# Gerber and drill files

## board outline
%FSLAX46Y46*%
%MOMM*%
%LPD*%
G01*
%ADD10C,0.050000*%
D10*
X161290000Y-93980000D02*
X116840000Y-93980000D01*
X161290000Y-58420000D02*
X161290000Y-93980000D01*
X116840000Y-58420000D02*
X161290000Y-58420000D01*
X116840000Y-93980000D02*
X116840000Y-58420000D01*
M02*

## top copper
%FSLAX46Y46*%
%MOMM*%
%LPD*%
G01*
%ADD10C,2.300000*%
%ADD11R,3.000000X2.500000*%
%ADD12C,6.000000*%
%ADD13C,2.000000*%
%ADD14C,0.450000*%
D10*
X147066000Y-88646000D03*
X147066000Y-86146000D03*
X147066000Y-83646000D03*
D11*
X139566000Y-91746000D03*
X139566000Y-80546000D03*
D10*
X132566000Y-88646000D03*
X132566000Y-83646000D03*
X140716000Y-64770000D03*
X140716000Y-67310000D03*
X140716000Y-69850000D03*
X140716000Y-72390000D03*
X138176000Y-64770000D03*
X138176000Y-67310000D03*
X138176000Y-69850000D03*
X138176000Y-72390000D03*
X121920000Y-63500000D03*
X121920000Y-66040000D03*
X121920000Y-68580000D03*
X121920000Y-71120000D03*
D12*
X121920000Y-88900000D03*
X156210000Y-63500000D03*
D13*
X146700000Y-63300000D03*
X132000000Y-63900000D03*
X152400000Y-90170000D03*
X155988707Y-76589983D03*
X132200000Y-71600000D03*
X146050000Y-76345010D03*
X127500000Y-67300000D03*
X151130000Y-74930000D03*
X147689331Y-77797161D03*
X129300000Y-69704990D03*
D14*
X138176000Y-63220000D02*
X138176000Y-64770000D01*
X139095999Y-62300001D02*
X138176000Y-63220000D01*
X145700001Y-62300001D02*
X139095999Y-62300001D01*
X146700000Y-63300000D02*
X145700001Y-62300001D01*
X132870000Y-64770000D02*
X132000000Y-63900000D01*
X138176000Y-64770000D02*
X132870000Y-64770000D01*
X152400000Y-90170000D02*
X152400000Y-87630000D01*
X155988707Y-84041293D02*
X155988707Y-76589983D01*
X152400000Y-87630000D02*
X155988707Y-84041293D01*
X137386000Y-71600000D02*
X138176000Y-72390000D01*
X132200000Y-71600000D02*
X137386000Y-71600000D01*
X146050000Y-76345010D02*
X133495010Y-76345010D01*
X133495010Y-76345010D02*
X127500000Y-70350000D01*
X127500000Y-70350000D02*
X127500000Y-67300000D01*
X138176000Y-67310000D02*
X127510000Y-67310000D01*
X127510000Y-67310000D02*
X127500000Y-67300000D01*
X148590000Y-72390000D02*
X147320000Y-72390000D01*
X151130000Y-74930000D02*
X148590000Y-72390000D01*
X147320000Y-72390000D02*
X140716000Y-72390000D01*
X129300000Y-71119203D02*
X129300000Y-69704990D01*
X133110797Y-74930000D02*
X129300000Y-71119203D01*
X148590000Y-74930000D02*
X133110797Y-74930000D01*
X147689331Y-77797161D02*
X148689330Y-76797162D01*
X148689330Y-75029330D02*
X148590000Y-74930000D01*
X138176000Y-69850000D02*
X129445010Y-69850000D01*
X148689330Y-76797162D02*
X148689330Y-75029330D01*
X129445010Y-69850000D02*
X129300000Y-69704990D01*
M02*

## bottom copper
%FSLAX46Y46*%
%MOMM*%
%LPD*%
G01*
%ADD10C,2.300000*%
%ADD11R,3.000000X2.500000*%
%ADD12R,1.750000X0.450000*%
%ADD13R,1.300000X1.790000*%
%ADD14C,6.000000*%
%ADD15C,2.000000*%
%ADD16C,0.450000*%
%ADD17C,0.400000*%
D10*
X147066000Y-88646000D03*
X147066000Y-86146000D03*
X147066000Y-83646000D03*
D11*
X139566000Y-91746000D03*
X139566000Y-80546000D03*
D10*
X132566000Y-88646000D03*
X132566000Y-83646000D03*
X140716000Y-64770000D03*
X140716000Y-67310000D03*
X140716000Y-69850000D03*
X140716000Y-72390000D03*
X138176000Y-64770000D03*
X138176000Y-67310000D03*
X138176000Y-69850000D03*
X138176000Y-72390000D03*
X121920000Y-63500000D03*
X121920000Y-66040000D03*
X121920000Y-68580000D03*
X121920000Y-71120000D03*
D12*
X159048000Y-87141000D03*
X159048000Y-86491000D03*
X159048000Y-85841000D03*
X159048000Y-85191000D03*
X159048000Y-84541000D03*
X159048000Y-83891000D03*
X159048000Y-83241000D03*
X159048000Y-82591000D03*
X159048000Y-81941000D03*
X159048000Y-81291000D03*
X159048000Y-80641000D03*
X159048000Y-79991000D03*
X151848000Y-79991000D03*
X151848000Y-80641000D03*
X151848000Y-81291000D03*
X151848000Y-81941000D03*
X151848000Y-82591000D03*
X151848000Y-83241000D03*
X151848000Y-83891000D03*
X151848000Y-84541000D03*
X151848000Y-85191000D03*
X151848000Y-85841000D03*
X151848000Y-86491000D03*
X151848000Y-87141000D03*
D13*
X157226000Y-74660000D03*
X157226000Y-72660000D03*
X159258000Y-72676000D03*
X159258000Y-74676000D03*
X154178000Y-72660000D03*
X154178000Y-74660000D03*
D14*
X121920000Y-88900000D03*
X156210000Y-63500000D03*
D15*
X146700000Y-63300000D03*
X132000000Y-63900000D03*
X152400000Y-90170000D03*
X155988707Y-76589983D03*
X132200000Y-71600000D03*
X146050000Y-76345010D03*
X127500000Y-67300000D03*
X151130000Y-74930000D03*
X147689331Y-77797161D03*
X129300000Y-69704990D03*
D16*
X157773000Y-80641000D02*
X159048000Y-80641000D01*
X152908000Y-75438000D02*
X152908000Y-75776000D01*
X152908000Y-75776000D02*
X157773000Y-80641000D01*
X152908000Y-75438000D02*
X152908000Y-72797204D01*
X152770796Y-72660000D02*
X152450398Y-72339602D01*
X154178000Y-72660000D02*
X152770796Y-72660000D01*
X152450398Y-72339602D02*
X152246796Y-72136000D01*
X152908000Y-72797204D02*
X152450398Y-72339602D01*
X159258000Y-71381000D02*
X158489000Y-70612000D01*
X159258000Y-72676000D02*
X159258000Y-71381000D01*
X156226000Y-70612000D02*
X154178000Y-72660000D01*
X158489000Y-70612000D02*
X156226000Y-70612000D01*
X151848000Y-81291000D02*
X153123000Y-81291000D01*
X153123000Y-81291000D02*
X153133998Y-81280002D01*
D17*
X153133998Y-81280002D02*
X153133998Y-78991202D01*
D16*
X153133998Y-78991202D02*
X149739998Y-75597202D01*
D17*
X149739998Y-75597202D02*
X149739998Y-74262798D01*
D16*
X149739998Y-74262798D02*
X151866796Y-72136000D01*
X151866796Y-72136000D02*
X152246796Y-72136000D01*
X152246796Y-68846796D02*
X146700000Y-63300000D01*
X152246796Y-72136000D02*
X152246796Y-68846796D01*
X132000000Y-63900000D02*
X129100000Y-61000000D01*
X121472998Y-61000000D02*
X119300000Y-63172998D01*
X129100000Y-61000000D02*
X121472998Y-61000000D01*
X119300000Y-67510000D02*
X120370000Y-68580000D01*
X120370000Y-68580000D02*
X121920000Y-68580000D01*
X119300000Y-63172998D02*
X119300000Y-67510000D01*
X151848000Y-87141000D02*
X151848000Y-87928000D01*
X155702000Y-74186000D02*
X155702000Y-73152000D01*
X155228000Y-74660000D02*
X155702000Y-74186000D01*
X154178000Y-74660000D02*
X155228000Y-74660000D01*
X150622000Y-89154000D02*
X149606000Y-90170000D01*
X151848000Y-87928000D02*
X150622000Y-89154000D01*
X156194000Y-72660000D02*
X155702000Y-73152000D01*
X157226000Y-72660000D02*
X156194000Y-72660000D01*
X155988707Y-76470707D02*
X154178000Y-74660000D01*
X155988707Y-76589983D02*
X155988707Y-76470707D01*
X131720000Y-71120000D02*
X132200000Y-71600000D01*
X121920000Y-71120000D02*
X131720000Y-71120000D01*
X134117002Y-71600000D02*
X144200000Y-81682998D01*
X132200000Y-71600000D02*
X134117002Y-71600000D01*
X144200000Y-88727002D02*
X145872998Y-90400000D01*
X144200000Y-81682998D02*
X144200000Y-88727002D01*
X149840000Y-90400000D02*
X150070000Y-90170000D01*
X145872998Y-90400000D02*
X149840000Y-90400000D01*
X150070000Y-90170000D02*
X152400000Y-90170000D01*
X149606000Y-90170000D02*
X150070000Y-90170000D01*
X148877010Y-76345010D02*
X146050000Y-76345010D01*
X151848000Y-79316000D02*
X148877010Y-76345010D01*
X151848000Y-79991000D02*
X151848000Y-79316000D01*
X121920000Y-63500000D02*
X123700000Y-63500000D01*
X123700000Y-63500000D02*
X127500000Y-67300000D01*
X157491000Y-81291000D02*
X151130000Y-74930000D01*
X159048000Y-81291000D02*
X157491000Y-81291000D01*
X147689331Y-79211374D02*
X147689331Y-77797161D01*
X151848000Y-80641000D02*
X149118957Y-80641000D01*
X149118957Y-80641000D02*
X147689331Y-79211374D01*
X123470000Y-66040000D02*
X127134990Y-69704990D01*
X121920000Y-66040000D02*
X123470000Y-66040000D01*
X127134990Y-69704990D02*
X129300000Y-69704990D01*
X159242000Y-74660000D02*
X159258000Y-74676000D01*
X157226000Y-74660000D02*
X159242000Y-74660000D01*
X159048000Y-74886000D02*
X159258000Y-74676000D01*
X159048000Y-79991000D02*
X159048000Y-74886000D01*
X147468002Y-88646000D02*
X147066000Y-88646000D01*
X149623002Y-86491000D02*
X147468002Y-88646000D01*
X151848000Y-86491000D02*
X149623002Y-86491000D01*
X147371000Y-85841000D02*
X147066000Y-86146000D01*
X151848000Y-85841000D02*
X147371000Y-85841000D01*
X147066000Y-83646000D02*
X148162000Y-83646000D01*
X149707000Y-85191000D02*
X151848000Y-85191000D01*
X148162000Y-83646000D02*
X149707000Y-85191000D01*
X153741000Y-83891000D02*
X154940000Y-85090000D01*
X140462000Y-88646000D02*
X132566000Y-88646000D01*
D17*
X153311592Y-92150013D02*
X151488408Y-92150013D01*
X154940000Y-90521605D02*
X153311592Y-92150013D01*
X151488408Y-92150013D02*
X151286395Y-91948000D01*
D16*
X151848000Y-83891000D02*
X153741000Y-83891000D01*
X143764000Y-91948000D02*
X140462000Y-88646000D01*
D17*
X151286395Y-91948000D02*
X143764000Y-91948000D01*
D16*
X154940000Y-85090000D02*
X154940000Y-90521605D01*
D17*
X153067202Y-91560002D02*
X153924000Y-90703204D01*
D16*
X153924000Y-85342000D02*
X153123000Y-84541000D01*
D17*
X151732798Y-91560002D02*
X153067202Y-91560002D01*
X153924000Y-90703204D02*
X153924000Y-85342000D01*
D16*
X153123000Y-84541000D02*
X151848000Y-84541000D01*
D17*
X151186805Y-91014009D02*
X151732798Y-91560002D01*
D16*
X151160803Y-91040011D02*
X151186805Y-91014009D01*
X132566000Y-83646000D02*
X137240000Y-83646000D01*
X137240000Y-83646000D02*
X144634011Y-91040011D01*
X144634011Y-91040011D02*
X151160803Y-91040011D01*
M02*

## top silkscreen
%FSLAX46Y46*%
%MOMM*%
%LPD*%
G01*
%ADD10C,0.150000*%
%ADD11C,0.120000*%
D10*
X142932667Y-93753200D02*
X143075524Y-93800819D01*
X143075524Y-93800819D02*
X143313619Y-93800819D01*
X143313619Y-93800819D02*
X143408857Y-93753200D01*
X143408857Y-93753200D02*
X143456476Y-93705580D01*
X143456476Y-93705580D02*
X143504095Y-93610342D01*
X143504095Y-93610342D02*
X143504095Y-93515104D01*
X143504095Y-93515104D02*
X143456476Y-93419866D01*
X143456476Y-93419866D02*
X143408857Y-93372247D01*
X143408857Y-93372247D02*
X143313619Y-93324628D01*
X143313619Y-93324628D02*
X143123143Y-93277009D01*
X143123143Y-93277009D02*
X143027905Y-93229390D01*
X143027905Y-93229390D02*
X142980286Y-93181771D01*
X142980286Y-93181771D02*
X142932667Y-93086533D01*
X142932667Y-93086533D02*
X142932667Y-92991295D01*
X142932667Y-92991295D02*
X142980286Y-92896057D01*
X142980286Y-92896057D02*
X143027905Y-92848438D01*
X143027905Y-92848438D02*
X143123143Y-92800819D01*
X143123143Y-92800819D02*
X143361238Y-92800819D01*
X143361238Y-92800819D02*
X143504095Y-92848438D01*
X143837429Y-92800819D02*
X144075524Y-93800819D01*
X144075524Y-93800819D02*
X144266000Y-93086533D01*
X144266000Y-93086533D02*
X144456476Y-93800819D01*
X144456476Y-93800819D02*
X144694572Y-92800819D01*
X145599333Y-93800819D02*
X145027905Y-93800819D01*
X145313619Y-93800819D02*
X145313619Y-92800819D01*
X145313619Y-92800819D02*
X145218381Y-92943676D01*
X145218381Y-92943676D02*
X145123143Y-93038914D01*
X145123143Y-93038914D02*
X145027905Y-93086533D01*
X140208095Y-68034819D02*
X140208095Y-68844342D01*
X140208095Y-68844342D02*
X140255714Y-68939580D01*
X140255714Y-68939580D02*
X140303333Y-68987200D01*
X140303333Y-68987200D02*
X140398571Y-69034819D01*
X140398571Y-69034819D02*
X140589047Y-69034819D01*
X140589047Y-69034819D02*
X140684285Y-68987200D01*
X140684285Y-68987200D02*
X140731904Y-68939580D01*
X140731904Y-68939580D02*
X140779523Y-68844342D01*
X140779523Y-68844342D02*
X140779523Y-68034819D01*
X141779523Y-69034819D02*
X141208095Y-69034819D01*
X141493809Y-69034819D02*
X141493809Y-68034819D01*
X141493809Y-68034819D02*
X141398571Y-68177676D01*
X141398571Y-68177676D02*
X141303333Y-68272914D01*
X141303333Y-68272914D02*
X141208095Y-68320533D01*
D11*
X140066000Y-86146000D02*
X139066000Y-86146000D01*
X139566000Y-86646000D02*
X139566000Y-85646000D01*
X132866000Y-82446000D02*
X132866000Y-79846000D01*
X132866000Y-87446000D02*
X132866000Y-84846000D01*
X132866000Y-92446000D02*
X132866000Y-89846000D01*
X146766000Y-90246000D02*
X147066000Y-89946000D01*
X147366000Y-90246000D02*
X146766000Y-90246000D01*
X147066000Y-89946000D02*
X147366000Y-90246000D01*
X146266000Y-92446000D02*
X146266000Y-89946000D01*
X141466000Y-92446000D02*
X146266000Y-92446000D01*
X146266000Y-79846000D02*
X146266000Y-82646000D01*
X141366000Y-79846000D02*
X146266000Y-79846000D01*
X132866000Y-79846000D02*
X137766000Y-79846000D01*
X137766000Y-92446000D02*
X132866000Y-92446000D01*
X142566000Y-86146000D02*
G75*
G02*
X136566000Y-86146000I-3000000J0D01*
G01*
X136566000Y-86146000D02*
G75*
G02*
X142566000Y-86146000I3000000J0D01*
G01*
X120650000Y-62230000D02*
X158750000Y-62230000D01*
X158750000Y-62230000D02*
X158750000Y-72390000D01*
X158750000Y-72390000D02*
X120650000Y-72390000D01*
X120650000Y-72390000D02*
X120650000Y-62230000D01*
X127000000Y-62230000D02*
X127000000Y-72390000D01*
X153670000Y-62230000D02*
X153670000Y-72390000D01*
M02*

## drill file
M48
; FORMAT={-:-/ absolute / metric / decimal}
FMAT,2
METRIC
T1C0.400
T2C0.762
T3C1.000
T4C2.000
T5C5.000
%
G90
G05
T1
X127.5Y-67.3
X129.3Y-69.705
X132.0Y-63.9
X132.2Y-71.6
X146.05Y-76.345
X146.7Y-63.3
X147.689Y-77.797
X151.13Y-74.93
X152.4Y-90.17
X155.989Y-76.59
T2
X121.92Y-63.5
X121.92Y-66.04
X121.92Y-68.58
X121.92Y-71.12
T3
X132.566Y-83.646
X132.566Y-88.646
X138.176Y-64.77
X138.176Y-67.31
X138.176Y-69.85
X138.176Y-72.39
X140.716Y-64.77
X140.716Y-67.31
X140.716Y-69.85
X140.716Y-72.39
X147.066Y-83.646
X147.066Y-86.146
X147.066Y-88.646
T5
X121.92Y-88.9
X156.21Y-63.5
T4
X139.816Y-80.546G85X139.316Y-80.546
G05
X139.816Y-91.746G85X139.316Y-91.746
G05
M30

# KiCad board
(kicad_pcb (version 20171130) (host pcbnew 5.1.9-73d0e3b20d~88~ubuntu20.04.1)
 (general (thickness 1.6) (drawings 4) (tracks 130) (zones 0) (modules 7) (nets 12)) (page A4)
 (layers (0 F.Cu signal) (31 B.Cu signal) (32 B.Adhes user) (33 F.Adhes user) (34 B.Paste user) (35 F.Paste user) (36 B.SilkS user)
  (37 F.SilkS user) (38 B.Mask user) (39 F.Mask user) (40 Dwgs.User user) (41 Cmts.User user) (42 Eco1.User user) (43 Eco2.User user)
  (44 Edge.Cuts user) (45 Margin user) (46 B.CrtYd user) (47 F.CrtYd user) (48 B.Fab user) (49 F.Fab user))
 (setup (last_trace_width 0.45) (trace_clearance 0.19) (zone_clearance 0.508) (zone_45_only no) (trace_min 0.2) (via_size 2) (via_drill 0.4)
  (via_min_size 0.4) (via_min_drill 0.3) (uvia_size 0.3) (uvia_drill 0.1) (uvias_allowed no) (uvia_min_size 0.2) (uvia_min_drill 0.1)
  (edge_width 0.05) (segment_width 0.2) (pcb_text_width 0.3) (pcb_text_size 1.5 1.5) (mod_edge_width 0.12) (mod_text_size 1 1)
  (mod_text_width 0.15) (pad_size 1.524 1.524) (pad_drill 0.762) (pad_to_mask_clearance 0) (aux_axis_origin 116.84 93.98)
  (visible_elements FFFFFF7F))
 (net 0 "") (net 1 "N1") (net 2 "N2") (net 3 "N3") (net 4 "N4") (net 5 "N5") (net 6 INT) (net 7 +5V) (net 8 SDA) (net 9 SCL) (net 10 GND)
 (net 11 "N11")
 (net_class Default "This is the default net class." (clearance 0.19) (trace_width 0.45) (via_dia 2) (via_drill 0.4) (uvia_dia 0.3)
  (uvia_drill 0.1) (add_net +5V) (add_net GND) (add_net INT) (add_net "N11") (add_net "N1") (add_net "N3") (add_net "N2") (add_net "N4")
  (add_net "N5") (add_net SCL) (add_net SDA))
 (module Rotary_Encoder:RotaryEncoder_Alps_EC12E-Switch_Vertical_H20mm (layer F.Cu) (at 147.066 88.646 180)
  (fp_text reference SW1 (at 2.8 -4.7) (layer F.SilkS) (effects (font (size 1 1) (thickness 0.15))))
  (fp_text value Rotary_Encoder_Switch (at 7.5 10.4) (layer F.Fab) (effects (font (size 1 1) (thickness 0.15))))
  (fp_line (start 7 2.5) (end 8 2.5) (layer F.SilkS) (width 0.12))
  (fp_line (start 7.5 2) (end 7.5 3) (layer F.SilkS) (width 0.12))
  (fp_line (start 14.2 6.2) (end 14.2 8.8) (layer F.SilkS) (width 0.12))
  (fp_line (start 14.2 1.2) (end 14.2 3.8) (layer F.SilkS) (width 0.12))
  (fp_line (start 14.2 -3.8) (end 14.2 -1.2) (layer F.SilkS) (width 0.12))
  (fp_line (start 0.3 -1.6) (end 0 -1.3) (layer F.SilkS) (width 0.12))
  (fp_line (start -0.3 -1.6) (end 0.3 -1.6) (layer F.SilkS) (width 0.12))
  (fp_line (start 0 -1.3) (end -0.3 -1.6) (layer F.SilkS) (width 0.12))
  (fp_line (start 0.8 -3.8) (end 0.8 -1.3) (layer F.SilkS) (width 0.12))
  (fp_line (start 5.6 -3.8) (end 0.8 -3.8) (layer F.SilkS) (width 0.12))
  (fp_line (start 0.8 8.8) (end 0.8 6) (layer F.SilkS) (width 0.12))
  (fp_line (start 5.7 8.8) (end 0.8 8.8) (layer F.SilkS) (width 0.12))
  (fp_line (start 14.2 8.8) (end 9.3 8.8) (layer F.SilkS) (width 0.12))
  (fp_line (start 9.3 -3.8) (end 14.2 -3.8) (layer F.SilkS) (width 0.12))
  (fp_circle (center 7.5 2.5) (end 10.5 2.5) (layer F.SilkS) (width 0.12))
  (pad A thru_hole circle (at 0 0 180) (size 2.3 2.3) (drill 1) (layers *.Cu *.Mask) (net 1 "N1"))
  (pad C thru_hole circle (at 0 2.5 180) (size 2.3 2.3) (drill 1) (layers *.Cu *.Mask) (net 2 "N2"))
  (pad B thru_hole circle (at 0 5 180) (size 2.3 2.3) (drill 1) (layers *.Cu *.Mask) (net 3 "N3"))
  (pad MP thru_hole rect (at 7.5 -3.1 180) (size 3 2.5) (drill oval 2.5 2) (layers *.Cu *.Mask))
  (pad MP thru_hole rect (at 7.5 8.1 180) (size 3 2.5) (drill oval 2.5 2) (layers *.Cu *.Mask))
  (pad S1 thru_hole circle (at 14.5 0 180) (size 2.3 2.3) (drill 1) (layers *.Cu *.Mask) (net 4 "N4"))
  (pad S2 thru_hole circle (at 14.5 5 180) (size 2.3 2.3) (drill 1) (layers *.Cu *.Mask) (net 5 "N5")))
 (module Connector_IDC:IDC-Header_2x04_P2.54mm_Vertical (layer B.Cu) (at 138.176 72.39)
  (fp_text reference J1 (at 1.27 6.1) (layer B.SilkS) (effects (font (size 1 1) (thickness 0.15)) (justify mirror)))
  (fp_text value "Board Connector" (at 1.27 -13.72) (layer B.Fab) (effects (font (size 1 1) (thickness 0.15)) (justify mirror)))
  (pad 8 thru_hole circle (at 2.54 -7.62) (size 2.3 2.3) (drill 1) (layers *.Cu *.Mask))
  (pad 6 thru_hole circle (at 2.54 -5.08) (size 2.3 2.3) (drill 1) (layers *.Cu *.Mask))
  (pad 4 thru_hole circle (at 2.54 -2.54) (size 2.3 2.3) (drill 1) (layers *.Cu *.Mask))
  (pad 2 thru_hole circle (at 2.54 0) (size 2.3 2.3) (drill 1) (layers *.Cu *.Mask) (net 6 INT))
  (pad 7 thru_hole circle (at 0 -7.62) (size 2.3 2.3) (drill 1) (layers *.Cu *.Mask) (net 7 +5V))
  (pad 5 thru_hole circle (at 0 -5.08) (size 2.3 2.3) (drill 1) (layers *.Cu *.Mask) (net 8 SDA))
  (pad 3 thru_hole circle (at 0 -2.54) (size 2.3 2.3) (drill 1) (layers *.Cu *.Mask) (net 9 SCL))
  (pad 1 thru_hole circle (at 0 0) (size 2.3 2.3) (drill 1) (layers *.Cu *.Mask) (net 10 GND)))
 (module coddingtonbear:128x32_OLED (layer F.Cu) (at 129.54 68.58)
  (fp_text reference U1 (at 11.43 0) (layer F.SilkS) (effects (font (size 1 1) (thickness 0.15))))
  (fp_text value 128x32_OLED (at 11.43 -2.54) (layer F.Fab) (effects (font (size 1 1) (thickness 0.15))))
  (fp_line (start -8.89 -6.35) (end 29.21 -6.35) (layer F.SilkS) (width 0.12))
  (fp_line (start 29.21 -6.35) (end 29.21 3.81) (layer F.SilkS) (width 0.12))
  (fp_line (start 29.21 3.81) (end -8.89 3.81) (layer F.SilkS) (width 0.12))
  (fp_line (start -8.89 3.81) (end -8.89 -6.35) (layer F.SilkS) (width 0.12))
  (fp_line (start -2.54 -6.35) (end -2.54 3.81) (layer F.SilkS) (width 0.12))
  (fp_line (start 24.13 -6.35) (end 24.13 3.81) (layer F.SilkS) (width 0.12))
  (pad 4 thru_hole circle (at -7.62 -5.08) (size 2.3 2.3) (drill 0.762) (layers *.Cu *.Mask) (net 8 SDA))
  (pad 3 thru_hole circle (at -7.62 -2.54) (size 2.3 2.3) (drill 0.762) (layers *.Cu *.Mask) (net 9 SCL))
  (pad 2 thru_hole circle (at -7.62 0) (size 2.3 2.3) (drill 0.762) (layers *.Cu *.Mask) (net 7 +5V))
  (pad 1 thru_hole circle (at -7.62 2.54) (size 2.3 2.3) (drill 0.762) (layers *.Cu *.Mask) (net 10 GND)))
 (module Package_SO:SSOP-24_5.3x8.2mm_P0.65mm (layer B.Cu) (at 155.448 83.566)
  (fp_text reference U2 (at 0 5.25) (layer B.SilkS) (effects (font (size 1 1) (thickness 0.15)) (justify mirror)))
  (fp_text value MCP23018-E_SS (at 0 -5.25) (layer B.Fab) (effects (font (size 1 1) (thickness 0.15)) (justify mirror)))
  (pad 24 smd rect (at 3.6 3.575) (size 1.75 0.45) (layers B.Cu B.Paste B.Mask))
  (pad 23 smd rect (at 3.6 2.925) (size 1.75 0.45) (layers B.Cu B.Paste B.Mask))
  (pad 22 smd rect (at 3.6 2.275) (size 1.75 0.45) (layers B.Cu B.Paste B.Mask))
  (pad 21 smd rect (at 3.6 1.625) (size 1.75 0.45) (layers B.Cu B.Paste B.Mask))
  (pad 20 smd rect (at 3.6 0.975) (size 1.75 0.45) (layers B.Cu B.Paste B.Mask))
  (pad 19 smd rect (at 3.6 0.325) (size 1.75 0.45) (layers B.Cu B.Paste B.Mask))
  (pad 18 smd rect (at 3.6 -0.325) (size 1.75 0.45) (layers B.Cu B.Paste B.Mask))
  (pad 17 smd rect (at 3.6 -0.975) (size 1.75 0.45) (layers B.Cu B.Paste B.Mask))
  (pad 16 smd rect (at 3.6 -1.625) (size 1.75 0.45) (layers B.Cu B.Paste B.Mask))
  (pad 15 smd rect (at 3.6 -2.275) (size 1.75 0.45) (layers B.Cu B.Paste B.Mask) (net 6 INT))
  (pad 14 smd rect (at 3.6 -2.925) (size 1.75 0.45) (layers B.Cu B.Paste B.Mask) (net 7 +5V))
  (pad 13 smd rect (at 3.6 -3.575) (size 1.75 0.45) (layers B.Cu B.Paste B.Mask) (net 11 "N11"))
  (pad 12 smd rect (at -3.6 -3.575) (size 1.75 0.45) (layers B.Cu B.Paste B.Mask) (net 8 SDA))
  (pad 11 smd rect (at -3.6 -2.925) (size 1.75 0.45) (layers B.Cu B.Paste B.Mask) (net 9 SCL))
  (pad 10 smd rect (at -3.6 -2.275) (size 1.75 0.45) (layers B.Cu B.Paste B.Mask) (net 7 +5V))
  (pad 9 smd rect (at -3.6 -1.625) (size 1.75 0.45) (layers B.Cu B.Paste B.Mask))
  (pad 8 smd rect (at -3.6 -0.975) (size 1.75 0.45) (layers B.Cu B.Paste B.Mask))
  (pad 7 smd rect (at -3.6 -0.325) (size 1.75 0.45) (layers B.Cu B.Paste B.Mask))
  (pad 6 smd rect (at -3.6 0.325) (size 1.75 0.45) (layers B.Cu B.Paste B.Mask) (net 4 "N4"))
  (pad 5 smd rect (at -3.6 0.975) (size 1.75 0.45) (layers B.Cu B.Paste B.Mask) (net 5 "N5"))
  (pad 4 smd rect (at -3.6 1.625) (size 1.75 0.45) (layers B.Cu B.Paste B.Mask) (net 3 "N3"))
  (pad 3 smd rect (at -3.6 2.275) (size 1.75 0.45) (layers B.Cu B.Paste B.Mask) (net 2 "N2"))
  (pad 2 smd rect (at -3.6 2.925) (size 1.75 0.45) (layers B.Cu B.Paste B.Mask) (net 1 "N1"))
  (pad 1 smd rect (at -3.6 3.575) (size 1.75 0.45) (layers B.Cu B.Paste B.Mask) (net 10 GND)))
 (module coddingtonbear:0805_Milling (layer B.Cu) (at 157.226 73.66 90)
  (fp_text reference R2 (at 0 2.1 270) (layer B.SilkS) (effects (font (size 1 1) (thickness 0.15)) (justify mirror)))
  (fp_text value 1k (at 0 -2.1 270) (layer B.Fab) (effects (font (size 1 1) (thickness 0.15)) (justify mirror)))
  (pad 1 smd rect (at -1 0 90) (size 1.79 1.3) (layers B.Cu B.Paste B.Mask) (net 11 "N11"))
  (pad 2 smd rect (at 1 0 90) (size 1.79 1.3) (layers B.Cu B.Paste B.Mask) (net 10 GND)))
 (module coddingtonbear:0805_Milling (layer B.Cu) (at 159.258 73.676 270)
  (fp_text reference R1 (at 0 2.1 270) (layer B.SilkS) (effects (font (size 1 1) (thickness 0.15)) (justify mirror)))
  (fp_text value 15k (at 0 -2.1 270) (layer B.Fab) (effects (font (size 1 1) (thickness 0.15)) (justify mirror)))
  (pad 1 smd rect (at -1 0 270) (size 1.79 1.3) (layers B.Cu B.Paste B.Mask) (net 7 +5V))
  (pad 2 smd rect (at 1 0 270) (size 1.79 1.3) (layers B.Cu B.Paste B.Mask) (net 11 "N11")))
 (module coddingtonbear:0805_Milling (layer B.Cu) (at 154.178 73.66 270)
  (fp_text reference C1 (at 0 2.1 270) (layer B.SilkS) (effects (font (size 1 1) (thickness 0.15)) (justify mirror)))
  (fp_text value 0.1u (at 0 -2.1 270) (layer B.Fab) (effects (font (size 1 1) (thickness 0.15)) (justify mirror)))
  (pad 1 smd rect (at -1 0 270) (size 1.79 1.3) (layers B.Cu B.Paste B.Mask) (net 7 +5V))
  (pad 2 smd rect (at 1 0 270) (size 1.79 1.3) (layers B.Cu B.Paste B.Mask) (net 10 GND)))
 (gr_line (start 161.29 93.98) (end 116.84 93.98) (layer Edge.Cuts) (width 0.05))
 (gr_line (start 161.29 58.42) (end 161.29 93.98) (layer Edge.Cuts) (width 0.05))
 (gr_line (start 116.84 58.42) (end 161.29 58.42) (layer Edge.Cuts) (width 0.05))
 (gr_line (start 116.84 93.98) (end 116.84 58.42) (layer Edge.Cuts) (width 0.05))
 (via (at 121.92 88.9) (size 6) (drill 5) (layers F.Cu B.Cu) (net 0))
 (via (at 156.21 63.5) (size 6) (drill 5) (layers F.Cu B.Cu) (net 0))
 (segment (start 157.773 80.641) (end 159.048 80.641) (width 0.45) (layer B.Cu) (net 7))
 (segment (start 152.908 75.438) (end 152.908 75.776) (width 0.45) (layer B.Cu) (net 7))
 (segment (start 152.908 75.776) (end 157.773 80.641) (width 0.45) (layer B.Cu) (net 7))
 (segment (start 152.908 75.438) (end 152.908 72.797204) (width 0.45) (layer B.Cu) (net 7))
 (segment (start 152.770796 72.66) (end 152.450398 72.339602) (width 0.45) (layer B.Cu) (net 7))
 (segment (start 154.178 72.66) (end 152.770796 72.66) (width 0.45) (layer B.Cu) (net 7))
 (segment (start 152.450398 72.339602) (end 152.246796 72.136) (width 0.45) (layer B.Cu) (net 7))
 (segment (start 152.908 72.797204) (end 152.450398 72.339602) (width 0.45) (layer B.Cu) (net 7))
 (segment (start 159.258 71.381) (end 158.489 70.612) (width 0.45) (layer B.Cu) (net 7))
 (segment (start 159.258 72.676) (end 159.258 71.381) (width 0.45) (layer B.Cu) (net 7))
 (segment (start 156.226 70.612) (end 154.178 72.66) (width 0.45) (layer B.Cu) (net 7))
 (segment (start 158.489 70.612) (end 156.226 70.612) (width 0.45) (layer B.Cu) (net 7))
 (segment (start 151.848 81.291) (end 153.123 81.291) (width 0.45) (layer B.Cu) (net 7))
 (segment (start 153.123 81.291) (end 153.133998 81.280002) (width 0.45) (layer B.Cu) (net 7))
 (segment (start 153.133998 81.280002) (end 153.133998 78.991202) (width 0.4) (layer B.Cu) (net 7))
 (segment (start 153.133998 78.991202) (end 149.739998 75.597202) (width 0.45) (layer B.Cu) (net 7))
 (segment (start 149.739998 75.597202) (end 149.739998 74.262798) (width 0.4) (layer B.Cu) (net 7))
 (segment (start 149.739998 74.262798) (end 151.866796 72.136) (width 0.45) (layer B.Cu) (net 7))
 (segment (start 151.866796 72.136) (end 152.246796 72.136) (width 0.45) (layer B.Cu) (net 7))
 (via (at 146.7 63.3) (size 2) (drill 0.4) (layers F.Cu B.Cu) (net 7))
 (segment (start 152.246796 68.846796) (end 146.7 63.3) (width 0.45) (layer B.Cu) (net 7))
 (segment (start 152.246796 72.136) (end 152.246796 68.846796) (width 0.45) (layer B.Cu) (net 7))
 (segment (start 138.176 63.22) (end 138.176 64.77) (width 0.45) (layer F.Cu) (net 7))
 (segment (start 139.095999 62.300001) (end 138.176 63.22) (width 0.45) (layer F.Cu) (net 7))
 (segment (start 145.700001 62.300001) (end 139.095999 62.300001) (width 0.45) (layer F.Cu) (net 7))
 (segment (start 146.7 63.3) (end 145.700001 62.300001) (width 0.45) (layer F.Cu) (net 7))
 (segment (start 132.87 64.77) (end 132 63.9) (width 0.45) (layer F.Cu) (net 7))
 (via (at 132 63.9) (size 2) (drill 0.4) (layers F.Cu B.Cu) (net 7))
 (segment (start 138.176 64.77) (end 132.87 64.77) (width 0.45) (layer F.Cu) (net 7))
 (segment (start 132 63.9) (end 129.1 61) (width 0.45) (layer B.Cu) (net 7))
 (segment (start 121.472998 61) (end 119.3 63.172998) (width 0.45) (layer B.Cu) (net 7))
 (segment (start 129.1 61) (end 121.472998 61) (width 0.45) (layer B.Cu) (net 7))
 (segment (start 119.3 67.51) (end 120.37 68.58) (width 0.45) (layer B.Cu) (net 7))
 (segment (start 120.37 68.58) (end 121.92 68.58) (width 0.45) (layer B.Cu) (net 7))
 (segment (start 119.3 63.172998) (end 119.3 67.51) (width 0.45) (layer B.Cu) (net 7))
 (segment (start 151.848 87.141) (end 151.848 87.928) (width 0.45) (layer B.Cu) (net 10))
 (segment (start 155.702 74.186) (end 155.702 73.152) (width 0.45) (layer B.Cu) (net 10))
 (segment (start 155.228 74.66) (end 155.702 74.186) (width 0.45) (layer B.Cu) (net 10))
 (segment (start 154.178 74.66) (end 155.228 74.66) (width 0.45) (layer B.Cu) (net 10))
 (segment (start 150.622 89.154) (end 149.606 90.17) (width 0.45) (layer B.Cu) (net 10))
 (segment (start 151.848 87.928) (end 150.622 89.154) (width 0.45) (layer B.Cu) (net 10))
 (segment (start 156.194 72.66) (end 155.702 73.152) (width 0.45) (layer B.Cu) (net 10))
 (segment (start 157.226 72.66) (end 156.194 72.66) (width 0.45) (layer B.Cu) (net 10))
 (via (at 152.4 90.17) (size 2) (drill 0.4) (layers F.Cu B.Cu) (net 10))
 (segment (start 152.4 90.17) (end 152.4 87.63) (width 0.45) (layer F.Cu) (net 10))
 (via (at 155.988707 76.589983) (size 2) (drill 0.4) (layers F.Cu B.Cu) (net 10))
 (segment (start 155.988707 84.041293) (end 155.988707 76.589983) (width 0.45) (layer F.Cu) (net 10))
 (segment (start 152.4 87.63) (end 155.988707 84.041293) (width 0.45) (layer F.Cu) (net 10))
 (segment (start 155.988707 76.470707) (end 154.178 74.66) (width 0.45) (layer B.Cu) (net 10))
 (segment (start 155.988707 76.589983) (end 155.988707 76.470707) (width 0.45) (layer B.Cu) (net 10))
 (segment (start 131.72 71.12) (end 132.2 71.6) (width 0.45) (layer B.Cu) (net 10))
 (segment (start 121.92 71.12) (end 131.72 71.12) (width 0.45) (layer B.Cu) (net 10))
 (via (at 132.2 71.6) (size 2) (drill 0.4) (layers F.Cu B.Cu) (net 10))
 (segment (start 137.386 71.6) (end 138.176 72.39) (width 0.45) (layer F.Cu) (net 10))
 (segment (start 132.2 71.6) (end 137.386 71.6) (width 0.45) (layer F.Cu) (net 10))
 (segment (start 134.117002 71.6) (end 144.2 81.682998) (width 0.45) (layer B.Cu) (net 10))
 (segment (start 132.2 71.6) (end 134.117002 71.6) (width 0.45) (layer B.Cu) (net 10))
 (segment (start 144.2 88.727002) (end 145.872998 90.4) (width 0.45) (layer B.Cu) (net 10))
 (segment (start 144.2 81.682998) (end 144.2 88.727002) (width 0.45) (layer B.Cu) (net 10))
 (segment (start 149.84 90.4) (end 150.07 90.17) (width 0.45) (layer B.Cu) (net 10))
 (segment (start 145.872998 90.4) (end 149.84 90.4) (width 0.45) (layer B.Cu) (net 10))
 (segment (start 150.07 90.17) (end 152.4 90.17) (width 0.45) (layer B.Cu) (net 10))
 (segment (start 149.606 90.17) (end 150.07 90.17) (width 0.45) (layer B.Cu) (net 10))
 (segment (start 148.87701 76.34501) (end 146.05 76.34501) (width 0.45) (layer B.Cu) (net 8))
 (segment (start 151.848 79.316) (end 148.87701 76.34501) (width 0.45) (layer B.Cu) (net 8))
 (segment (start 151.848 79.991) (end 151.848 79.316) (width 0.45) (layer B.Cu) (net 8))
 (via (at 146.05 76.34501) (size 2) (drill 0.4) (layers F.Cu B.Cu) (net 8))
 (segment (start 121.92 63.5) (end 123.7 63.5) (width 0.45) (layer B.Cu) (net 8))
 (segment (start 123.7 63.5) (end 127.5 67.3) (width 0.45) (layer B.Cu) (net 8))
 (segment (start 146.05 76.34501) (end 133.49501 76.34501) (width 0.45) (layer F.Cu) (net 8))
 (via (at 127.5 67.3) (size 2) (drill 0.4) (layers F.Cu B.Cu) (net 8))
 (segment (start 133.49501 76.34501) (end 127.5 70.35) (width 0.45) (layer F.Cu) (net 8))
 (segment (start 127.5 70.35) (end 127.5 67.3) (width 0.45) (layer F.Cu) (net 8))
 (segment (start 138.176 67.31) (end 127.51 67.31) (width 0.45) (layer F.Cu) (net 8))
 (segment (start 127.51 67.31) (end 127.5 67.3) (width 0.45) (layer F.Cu) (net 8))
 (via (at 151.13 74.93) (size 2) (drill 0.4) (layers F.Cu B.Cu) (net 6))
 (segment (start 157.491 81.291) (end 151.13 74.93) (width 0.45) (layer B.Cu) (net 6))
 (segment (start 159.048 81.291) (end 157.491 81.291) (width 0.45) (layer B.Cu) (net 6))
 (segment (start 148.59 72.39) (end 147.32 72.39) (width 0.45) (layer F.Cu) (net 6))
 (segment (start 151.13 74.93) (end 148.59 72.39) (width 0.45) (layer F.Cu) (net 6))
 (segment (start 147.32 72.39) (end 140.716 72.39) (width 0.45) (layer F.Cu) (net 6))
 (segment (start 147.689331 79.211374) (end 147.689331 77.797161) (width 0.45) (layer B.Cu) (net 9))
 (via (at 147.689331 77.797161) (size 2) (drill 0.4) (layers F.Cu B.Cu) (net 9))
 (segment (start 151.848 80.641) (end 149.118957 80.641) (width 0.45) (layer B.Cu) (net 9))
 (segment (start 149.118957 80.641) (end 147.689331 79.211374) (width 0.45) (layer B.Cu) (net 9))
 (segment (start 129.3 71.119203) (end 129.3 69.70499) (width 0.45) (layer F.Cu) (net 9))
 (segment (start 133.110797 74.93) (end 129.3 71.119203) (width 0.45) (layer F.Cu) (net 9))
 (segment (start 148.59 74.93) (end 133.110797 74.93) (width 0.45) (layer F.Cu) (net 9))
 (segment (start 147.689331 77.797161) (end 148.68933 76.797162) (width 0.45) (layer F.Cu) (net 9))
 (segment (start 148.68933 75.02933) (end 148.59 74.93) (width 0.45) (layer F.Cu) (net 9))
 (segment (start 138.176 69.85) (end 129.44501 69.85) (width 0.45) (layer F.Cu) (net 9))
 (segment (start 148.68933 76.797162) (end 148.68933 75.02933) (width 0.45) (layer F.Cu) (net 9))
 (segment (start 123.47 66.04) (end 127.13499 69.70499) (width 0.45) (layer B.Cu) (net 9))
 (segment (start 129.44501 69.85) (end 129.3 69.70499) (width 0.45) (layer F.Cu) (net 9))
 (segment (start 121.92 66.04) (end 123.47 66.04) (width 0.45) (layer B.Cu) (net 9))
 (via (at 129.3 69.70499) (size 2) (drill 0.4) (layers F.Cu B.Cu) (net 9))
 (segment (start 127.13499 69.70499) (end 129.3 69.70499) (width 0.45) (layer B.Cu) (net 9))
 (segment (start 159.242 74.66) (end 159.258 74.676) (width 0.45) (layer B.Cu) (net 11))
 (segment (start 157.226 74.66) (end 159.242 74.66) (width 0.45) (layer B.Cu) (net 11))
 (segment (start 159.048 74.886) (end 159.258 74.676) (width 0.45) (layer B.Cu) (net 11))
 (segment (start 159.048 79.991) (end 159.048 74.886) (width 0.45) (layer B.Cu) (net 11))
 (segment (start 147.468002 88.646) (end 147.066 88.646) (width 0.45) (layer B.Cu) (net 1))
 (segment (start 149.623002 86.491) (end 147.468002 88.646) (width 0.45) (layer B.Cu) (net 1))
 (segment (start 151.848 86.491) (end 149.623002 86.491) (width 0.45) (layer B.Cu) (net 1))
 (segment (start 147.371 85.841) (end 147.066 86.146) (width 0.45) (layer B.Cu) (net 2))
 (segment (start 151.848 85.841) (end 147.371 85.841) (width 0.45) (layer B.Cu) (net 2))
 (segment (start 147.066 83.646) (end 148.162 83.646) (width 0.45) (layer B.Cu) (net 3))
 (segment (start 149.707 85.191) (end 151.848 85.191) (width 0.45) (layer B.Cu) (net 3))
 (segment (start 148.162 83.646) (end 149.707 85.191) (width 0.45) (layer B.Cu) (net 3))
 (segment (start 153.741 83.891) (end 154.94 85.09) (width 0.45) (layer B.Cu) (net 4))
 (segment (start 140.462 88.646) (end 132.566 88.646) (width 0.45) (layer B.Cu) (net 4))
 (segment (start 153.311592 92.150013) (end 151.488408 92.150013) (width 0.4) (layer B.Cu) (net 4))
 (segment (start 154.94 90.521605) (end 153.311592 92.150013) (width 0.4) (layer B.Cu) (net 4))
 (segment (start 151.488408 92.150013) (end 151.286395 91.948) (width 0.4) (layer B.Cu) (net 4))
 (segment (start 151.848 83.891) (end 153.741 83.891) (width 0.45) (layer B.Cu) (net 4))
 (segment (start 143.764 91.948) (end 140.462 88.646) (width 0.45) (layer B.Cu) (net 4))
 (segment (start 151.286395 91.948) (end 143.764 91.948) (width 0.4) (layer B.Cu) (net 4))
 (segment (start 154.94 85.09) (end 154.94 90.521605) (width 0.45) (layer B.Cu) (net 4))
 (segment (start 153.067202 91.560002) (end 153.924 90.703204) (width 0.4) (layer B.Cu) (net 5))
 (segment (start 153.924 85.342) (end 153.123 84.541) (width 0.45) (layer B.Cu) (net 5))
 (segment (start 151.732798 91.560002) (end 153.067202 91.560002) (width 0.4) (layer B.Cu) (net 5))
 (segment (start 153.924 90.703204) (end 153.924 85.342) (width 0.4) (layer B.Cu) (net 5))
 (segment (start 153.123 84.541) (end 151.848 84.541) (width 0.45) (layer B.Cu) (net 5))
 (segment (start 151.186805 91.014009) (end 151.732798 91.560002) (width 0.4) (layer B.Cu) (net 5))
 (segment (start 151.160803 91.040011) (end 151.186805 91.014009) (width 0.45) (layer B.Cu) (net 5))
 (segment (start 132.566 83.646) (end 137.24 83.646) (width 0.45) (layer B.Cu) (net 5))
 (segment (start 137.24 83.646) (end 144.634011 91.040011) (width 0.45) (layer B.Cu) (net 5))
 (segment (start 144.634011 91.040011) (end 151.160803 91.040011) (width 0.45) (layer B.Cu) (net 5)))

